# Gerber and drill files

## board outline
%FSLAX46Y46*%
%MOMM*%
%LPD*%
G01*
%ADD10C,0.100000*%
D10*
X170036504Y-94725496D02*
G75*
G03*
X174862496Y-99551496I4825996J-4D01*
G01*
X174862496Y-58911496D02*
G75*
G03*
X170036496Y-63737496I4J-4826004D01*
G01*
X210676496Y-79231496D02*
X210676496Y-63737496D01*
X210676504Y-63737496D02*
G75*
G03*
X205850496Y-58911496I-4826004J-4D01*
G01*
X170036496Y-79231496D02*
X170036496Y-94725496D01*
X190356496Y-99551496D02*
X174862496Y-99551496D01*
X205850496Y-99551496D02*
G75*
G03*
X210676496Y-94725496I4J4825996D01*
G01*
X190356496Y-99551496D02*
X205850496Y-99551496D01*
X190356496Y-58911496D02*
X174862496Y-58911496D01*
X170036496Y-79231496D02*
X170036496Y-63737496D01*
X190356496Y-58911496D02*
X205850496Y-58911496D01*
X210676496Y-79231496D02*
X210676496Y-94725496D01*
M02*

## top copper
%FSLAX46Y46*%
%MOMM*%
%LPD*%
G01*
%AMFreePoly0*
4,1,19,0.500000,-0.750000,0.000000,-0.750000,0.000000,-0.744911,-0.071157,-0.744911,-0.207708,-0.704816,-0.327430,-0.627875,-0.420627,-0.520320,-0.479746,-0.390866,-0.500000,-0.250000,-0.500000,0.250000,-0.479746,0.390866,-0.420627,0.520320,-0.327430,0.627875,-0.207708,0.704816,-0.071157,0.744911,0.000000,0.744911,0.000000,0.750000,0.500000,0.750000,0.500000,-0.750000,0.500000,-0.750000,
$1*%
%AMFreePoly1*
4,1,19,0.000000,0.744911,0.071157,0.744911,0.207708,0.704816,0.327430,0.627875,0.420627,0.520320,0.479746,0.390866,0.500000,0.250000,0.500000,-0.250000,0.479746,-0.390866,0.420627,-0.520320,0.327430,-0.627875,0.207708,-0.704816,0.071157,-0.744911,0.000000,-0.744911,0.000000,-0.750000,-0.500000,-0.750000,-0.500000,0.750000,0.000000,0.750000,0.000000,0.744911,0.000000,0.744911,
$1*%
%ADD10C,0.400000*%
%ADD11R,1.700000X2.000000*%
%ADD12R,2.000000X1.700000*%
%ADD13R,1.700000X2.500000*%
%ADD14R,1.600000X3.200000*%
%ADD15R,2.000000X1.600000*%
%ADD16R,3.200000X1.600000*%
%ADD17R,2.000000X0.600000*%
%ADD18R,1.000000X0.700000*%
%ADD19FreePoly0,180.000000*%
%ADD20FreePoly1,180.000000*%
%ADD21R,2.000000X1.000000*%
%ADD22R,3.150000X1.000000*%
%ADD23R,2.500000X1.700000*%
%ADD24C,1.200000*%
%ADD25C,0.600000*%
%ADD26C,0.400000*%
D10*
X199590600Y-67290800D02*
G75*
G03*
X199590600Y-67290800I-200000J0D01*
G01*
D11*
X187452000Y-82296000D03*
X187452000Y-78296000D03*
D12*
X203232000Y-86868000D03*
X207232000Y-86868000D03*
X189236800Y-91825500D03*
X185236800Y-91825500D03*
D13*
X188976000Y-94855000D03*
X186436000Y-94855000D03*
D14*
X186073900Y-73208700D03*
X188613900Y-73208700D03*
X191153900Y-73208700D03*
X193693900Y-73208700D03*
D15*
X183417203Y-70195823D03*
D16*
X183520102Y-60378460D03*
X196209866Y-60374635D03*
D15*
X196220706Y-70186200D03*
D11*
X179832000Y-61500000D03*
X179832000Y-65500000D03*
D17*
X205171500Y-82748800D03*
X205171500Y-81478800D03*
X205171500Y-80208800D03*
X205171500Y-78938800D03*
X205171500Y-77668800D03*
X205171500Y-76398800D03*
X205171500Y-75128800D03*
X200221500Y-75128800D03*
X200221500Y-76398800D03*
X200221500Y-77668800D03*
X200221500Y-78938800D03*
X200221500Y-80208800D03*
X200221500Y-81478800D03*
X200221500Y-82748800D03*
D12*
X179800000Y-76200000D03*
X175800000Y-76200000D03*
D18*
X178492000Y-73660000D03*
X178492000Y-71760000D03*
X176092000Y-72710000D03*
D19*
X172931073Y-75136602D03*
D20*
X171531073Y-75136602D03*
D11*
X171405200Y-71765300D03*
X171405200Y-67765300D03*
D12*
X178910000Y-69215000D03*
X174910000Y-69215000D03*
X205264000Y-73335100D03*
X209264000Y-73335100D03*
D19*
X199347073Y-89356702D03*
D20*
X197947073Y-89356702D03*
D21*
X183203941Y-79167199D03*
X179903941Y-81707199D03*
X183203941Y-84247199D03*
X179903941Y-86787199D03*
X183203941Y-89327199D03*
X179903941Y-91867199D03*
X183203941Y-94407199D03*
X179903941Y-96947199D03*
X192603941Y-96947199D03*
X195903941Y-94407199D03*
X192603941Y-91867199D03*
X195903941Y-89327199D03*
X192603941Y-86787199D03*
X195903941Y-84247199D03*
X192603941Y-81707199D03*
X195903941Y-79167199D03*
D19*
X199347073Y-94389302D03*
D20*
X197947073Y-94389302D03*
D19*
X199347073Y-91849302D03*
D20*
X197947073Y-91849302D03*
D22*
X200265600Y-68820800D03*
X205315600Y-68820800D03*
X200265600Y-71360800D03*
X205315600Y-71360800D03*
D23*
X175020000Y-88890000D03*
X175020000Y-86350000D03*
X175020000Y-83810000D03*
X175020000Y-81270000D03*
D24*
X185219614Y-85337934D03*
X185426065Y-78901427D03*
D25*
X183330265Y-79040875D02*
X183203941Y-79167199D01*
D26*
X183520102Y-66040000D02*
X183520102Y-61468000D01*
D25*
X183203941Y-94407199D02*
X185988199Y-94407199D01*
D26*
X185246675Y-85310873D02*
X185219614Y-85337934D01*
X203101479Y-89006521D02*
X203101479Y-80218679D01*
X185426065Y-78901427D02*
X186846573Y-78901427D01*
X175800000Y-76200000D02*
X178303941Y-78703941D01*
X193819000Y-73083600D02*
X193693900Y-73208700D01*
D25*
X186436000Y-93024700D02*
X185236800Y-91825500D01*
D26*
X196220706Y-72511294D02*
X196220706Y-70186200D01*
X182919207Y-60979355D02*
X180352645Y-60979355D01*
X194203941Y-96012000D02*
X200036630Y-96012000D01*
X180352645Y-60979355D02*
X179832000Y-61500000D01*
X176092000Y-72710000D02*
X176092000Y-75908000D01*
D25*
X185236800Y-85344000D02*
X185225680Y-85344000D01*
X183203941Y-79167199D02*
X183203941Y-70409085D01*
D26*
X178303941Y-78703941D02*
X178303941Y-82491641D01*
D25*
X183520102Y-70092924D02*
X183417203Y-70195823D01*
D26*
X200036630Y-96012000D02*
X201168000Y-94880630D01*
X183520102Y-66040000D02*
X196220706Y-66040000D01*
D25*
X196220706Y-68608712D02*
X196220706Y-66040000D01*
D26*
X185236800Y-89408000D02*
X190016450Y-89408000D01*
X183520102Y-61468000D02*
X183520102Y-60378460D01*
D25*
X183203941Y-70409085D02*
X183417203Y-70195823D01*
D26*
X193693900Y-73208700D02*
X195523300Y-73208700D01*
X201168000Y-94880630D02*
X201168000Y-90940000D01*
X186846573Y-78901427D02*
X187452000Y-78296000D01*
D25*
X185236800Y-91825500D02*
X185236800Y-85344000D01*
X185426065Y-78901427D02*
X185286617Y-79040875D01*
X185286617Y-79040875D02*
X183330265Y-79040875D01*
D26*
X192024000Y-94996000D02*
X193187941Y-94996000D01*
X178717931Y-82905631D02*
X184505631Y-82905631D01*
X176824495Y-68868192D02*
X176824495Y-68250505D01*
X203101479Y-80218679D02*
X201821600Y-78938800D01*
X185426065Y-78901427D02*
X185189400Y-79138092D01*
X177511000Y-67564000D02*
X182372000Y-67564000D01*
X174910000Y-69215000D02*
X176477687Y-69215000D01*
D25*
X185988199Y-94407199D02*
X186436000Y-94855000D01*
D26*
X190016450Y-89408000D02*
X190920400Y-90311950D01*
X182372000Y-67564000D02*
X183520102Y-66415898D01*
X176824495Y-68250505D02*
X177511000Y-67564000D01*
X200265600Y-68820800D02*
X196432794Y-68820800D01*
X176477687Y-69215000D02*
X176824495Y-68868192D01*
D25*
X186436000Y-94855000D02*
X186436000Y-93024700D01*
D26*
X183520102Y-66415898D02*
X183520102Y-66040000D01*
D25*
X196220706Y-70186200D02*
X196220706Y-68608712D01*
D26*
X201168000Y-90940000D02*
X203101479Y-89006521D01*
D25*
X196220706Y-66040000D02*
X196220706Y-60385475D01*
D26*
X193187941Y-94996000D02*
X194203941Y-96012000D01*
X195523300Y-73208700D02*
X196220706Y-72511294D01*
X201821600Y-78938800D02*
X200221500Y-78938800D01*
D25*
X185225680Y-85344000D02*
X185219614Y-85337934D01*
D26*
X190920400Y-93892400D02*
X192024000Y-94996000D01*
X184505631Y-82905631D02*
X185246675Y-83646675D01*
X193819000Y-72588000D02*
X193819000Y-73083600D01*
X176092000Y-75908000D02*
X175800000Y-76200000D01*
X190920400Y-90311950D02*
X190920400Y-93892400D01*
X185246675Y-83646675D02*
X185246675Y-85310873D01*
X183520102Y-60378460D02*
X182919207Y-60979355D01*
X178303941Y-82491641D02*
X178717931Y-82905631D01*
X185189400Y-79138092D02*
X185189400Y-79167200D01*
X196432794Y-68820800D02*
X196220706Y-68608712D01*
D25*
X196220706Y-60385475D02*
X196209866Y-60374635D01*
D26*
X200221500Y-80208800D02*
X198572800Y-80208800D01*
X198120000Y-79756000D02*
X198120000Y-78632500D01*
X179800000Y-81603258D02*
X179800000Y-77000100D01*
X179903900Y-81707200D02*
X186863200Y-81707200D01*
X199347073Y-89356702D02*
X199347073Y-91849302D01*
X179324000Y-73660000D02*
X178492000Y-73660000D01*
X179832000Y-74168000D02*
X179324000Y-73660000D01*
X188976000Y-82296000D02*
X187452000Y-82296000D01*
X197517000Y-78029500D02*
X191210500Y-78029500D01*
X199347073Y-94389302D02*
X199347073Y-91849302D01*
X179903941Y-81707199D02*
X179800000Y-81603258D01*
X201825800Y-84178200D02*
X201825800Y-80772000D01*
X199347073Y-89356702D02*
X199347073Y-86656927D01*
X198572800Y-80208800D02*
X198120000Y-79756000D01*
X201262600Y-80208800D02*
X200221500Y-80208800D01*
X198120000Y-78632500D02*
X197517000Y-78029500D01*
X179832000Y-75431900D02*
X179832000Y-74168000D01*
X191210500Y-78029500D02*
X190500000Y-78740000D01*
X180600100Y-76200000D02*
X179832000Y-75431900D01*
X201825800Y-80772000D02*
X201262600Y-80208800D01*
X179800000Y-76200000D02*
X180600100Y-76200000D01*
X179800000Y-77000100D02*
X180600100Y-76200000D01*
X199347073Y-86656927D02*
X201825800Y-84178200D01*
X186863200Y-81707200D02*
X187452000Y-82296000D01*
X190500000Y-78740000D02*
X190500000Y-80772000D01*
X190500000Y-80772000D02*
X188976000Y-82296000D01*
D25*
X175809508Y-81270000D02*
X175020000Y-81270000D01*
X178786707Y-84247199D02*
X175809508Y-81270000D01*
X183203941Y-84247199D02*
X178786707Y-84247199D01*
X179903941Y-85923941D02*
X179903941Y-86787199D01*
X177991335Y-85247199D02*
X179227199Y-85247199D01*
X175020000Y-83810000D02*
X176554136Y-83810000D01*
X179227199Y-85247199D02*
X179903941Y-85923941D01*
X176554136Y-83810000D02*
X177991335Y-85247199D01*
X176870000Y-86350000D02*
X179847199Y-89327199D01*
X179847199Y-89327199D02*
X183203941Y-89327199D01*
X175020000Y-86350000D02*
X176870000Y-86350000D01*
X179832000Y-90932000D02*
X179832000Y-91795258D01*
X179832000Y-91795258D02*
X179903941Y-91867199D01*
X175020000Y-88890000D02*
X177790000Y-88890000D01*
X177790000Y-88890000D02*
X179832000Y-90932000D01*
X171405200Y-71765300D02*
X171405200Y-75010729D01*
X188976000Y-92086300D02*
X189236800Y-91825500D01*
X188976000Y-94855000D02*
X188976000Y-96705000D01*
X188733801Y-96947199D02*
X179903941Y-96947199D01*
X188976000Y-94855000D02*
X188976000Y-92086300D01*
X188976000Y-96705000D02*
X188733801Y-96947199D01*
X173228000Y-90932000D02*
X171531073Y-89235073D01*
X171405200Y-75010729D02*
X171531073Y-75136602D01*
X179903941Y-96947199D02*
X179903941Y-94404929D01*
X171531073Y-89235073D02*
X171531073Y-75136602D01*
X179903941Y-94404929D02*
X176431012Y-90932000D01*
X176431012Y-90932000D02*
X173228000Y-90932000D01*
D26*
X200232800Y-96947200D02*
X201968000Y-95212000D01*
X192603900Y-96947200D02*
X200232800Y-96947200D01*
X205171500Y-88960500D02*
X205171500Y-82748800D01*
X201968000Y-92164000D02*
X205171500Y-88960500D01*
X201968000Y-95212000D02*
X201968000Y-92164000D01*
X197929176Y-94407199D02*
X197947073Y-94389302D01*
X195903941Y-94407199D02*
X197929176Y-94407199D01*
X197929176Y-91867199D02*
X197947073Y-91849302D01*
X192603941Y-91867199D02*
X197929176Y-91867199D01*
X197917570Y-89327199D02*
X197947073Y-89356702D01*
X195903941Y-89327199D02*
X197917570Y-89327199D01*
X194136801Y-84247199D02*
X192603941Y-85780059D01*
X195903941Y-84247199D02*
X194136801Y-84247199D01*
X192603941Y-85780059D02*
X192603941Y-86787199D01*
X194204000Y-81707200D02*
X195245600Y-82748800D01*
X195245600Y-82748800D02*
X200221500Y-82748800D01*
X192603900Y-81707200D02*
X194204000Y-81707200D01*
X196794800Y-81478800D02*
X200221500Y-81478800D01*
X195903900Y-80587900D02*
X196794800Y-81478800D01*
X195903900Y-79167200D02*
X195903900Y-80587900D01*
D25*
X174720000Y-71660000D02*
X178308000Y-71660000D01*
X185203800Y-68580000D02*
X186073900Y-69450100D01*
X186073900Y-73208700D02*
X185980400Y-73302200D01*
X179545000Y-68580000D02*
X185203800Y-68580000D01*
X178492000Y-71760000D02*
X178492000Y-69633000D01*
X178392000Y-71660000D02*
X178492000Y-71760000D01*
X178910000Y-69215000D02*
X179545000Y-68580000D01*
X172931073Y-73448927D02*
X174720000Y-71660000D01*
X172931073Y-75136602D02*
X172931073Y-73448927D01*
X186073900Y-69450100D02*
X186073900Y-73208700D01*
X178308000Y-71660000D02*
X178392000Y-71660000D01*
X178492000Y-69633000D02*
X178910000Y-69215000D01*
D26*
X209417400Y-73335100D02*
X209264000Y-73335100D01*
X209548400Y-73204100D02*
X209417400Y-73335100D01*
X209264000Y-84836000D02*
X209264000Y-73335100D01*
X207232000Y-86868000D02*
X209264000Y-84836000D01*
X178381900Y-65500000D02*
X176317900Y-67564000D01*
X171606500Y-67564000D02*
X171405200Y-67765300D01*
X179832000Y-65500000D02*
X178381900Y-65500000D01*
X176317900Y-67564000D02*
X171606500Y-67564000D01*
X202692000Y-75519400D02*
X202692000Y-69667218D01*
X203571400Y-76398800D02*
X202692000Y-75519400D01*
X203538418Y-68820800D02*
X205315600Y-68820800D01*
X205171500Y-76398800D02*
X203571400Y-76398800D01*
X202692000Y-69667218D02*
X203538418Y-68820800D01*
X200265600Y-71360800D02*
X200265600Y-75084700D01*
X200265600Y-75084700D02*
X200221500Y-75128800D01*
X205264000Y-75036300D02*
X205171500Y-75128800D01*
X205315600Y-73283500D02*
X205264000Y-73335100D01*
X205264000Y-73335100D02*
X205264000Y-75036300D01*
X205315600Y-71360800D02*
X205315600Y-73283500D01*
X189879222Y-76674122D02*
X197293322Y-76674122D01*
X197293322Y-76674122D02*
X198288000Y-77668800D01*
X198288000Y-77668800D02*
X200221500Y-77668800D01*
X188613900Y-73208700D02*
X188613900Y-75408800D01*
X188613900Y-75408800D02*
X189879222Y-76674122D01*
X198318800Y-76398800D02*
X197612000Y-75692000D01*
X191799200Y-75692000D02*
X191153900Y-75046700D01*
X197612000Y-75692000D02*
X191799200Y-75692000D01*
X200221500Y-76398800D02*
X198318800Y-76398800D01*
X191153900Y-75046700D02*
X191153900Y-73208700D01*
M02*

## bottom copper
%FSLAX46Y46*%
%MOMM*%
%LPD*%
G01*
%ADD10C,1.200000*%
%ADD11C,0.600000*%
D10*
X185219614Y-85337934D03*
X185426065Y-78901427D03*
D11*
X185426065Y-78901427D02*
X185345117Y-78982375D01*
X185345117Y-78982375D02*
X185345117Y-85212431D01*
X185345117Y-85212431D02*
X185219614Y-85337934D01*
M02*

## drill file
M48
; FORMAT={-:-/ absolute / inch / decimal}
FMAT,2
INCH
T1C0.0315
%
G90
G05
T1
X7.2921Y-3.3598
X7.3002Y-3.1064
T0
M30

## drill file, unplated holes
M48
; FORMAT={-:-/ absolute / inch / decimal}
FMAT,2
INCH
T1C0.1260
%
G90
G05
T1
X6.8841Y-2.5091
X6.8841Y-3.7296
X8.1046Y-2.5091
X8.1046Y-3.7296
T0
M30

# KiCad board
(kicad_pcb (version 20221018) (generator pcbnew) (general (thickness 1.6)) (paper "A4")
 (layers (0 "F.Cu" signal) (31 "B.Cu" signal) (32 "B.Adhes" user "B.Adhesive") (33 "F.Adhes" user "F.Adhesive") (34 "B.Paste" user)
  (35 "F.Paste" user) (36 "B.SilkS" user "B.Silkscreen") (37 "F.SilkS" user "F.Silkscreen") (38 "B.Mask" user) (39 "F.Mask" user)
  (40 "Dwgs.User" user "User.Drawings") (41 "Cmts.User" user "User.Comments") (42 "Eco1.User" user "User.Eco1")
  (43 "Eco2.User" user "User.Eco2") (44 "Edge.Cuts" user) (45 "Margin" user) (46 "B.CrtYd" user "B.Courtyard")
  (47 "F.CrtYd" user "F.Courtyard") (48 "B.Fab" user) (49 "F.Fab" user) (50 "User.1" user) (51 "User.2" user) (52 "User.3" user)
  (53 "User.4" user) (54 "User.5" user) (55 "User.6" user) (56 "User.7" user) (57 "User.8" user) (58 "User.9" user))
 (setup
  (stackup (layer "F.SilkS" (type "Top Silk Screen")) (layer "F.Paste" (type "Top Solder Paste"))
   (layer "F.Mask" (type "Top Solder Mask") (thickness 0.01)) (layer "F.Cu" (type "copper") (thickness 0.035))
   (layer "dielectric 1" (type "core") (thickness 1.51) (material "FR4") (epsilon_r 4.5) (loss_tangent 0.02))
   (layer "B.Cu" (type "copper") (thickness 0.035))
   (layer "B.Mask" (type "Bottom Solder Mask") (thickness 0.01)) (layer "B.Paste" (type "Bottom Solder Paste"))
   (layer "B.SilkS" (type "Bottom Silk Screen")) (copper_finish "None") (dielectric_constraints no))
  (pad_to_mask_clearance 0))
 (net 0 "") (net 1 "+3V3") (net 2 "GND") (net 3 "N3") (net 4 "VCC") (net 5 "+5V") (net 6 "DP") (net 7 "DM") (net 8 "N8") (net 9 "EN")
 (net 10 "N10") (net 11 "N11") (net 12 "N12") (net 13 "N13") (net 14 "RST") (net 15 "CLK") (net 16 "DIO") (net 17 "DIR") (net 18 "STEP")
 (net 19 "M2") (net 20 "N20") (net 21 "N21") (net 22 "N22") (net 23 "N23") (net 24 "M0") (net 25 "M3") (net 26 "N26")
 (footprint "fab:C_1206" (layer "F.Cu") (at 187.452 80.296 90)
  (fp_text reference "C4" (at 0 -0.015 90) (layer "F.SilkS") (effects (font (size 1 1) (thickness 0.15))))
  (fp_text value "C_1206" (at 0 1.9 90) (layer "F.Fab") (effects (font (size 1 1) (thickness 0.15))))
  (pad "1" smd rect (at -2 0 90) (size 2 1.7) (layers "F.Cu" "F.Paste" "F.Mask") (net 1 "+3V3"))
  (pad "2" smd rect (at 2 0 90) (size 2 1.7) (layers "F.Cu" "F.Paste" "F.Mask") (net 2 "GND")))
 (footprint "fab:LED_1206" (layer "F.Cu") (at 205.232 86.868)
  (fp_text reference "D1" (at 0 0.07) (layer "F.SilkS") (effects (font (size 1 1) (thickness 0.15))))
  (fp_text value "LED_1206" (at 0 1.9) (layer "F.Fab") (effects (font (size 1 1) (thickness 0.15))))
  (pad "1" smd rect (at -2 0) (size 2 1.7) (layers "F.Cu" "F.Paste" "F.Mask") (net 2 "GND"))
  (pad "2" smd rect (at 2 0) (size 2 1.7) (layers "F.Cu" "F.Paste" "F.Mask") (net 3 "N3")))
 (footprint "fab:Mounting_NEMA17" (layer "F.Cu") (at 190.3565 79.2315)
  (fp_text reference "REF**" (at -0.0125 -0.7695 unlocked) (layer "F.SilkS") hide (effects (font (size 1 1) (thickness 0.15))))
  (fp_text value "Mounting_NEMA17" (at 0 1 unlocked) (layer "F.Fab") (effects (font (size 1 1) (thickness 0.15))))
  (pad "" np_thru_hole circle (at -15.5 -15.5) (size 3.2 3.2) (drill 3.2) (layers "*.Cu" "*.Mask") (clearance 1.9))
  (pad "" np_thru_hole circle (at -15.5 15.5) (size 3.2 3.2) (drill 3.2) (layers "*.Cu" "*.Mask") (clearance 1.9))
  (pad "" np_thru_hole circle (at 15.5 -15.5) (size 3.2 3.2) (drill 3.2) (layers "*.Cu" "*.Mask") (clearance 1.9))
  (pad "" np_thru_hole circle (at 15.5 15.5) (size 3.2 3.2) (drill 3.2) (layers "*.Cu" "*.Mask") (clearance 1.9)))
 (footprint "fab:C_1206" (layer "F.Cu") (at 187.2368 91.8255 180)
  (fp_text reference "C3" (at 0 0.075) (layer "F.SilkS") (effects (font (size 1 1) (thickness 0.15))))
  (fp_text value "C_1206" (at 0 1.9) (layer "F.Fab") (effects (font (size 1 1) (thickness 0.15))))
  (pad "1" smd rect (at -2 0 180) (size 2 1.7) (layers "F.Cu" "F.Paste" "F.Mask") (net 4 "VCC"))
  (pad "2" smd rect (at 2 0 180) (size 2 1.7) (layers "F.Cu" "F.Paste" "F.Mask") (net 2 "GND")))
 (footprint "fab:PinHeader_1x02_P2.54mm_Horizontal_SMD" (layer "F.Cu") (at 188.976 94.855 -90)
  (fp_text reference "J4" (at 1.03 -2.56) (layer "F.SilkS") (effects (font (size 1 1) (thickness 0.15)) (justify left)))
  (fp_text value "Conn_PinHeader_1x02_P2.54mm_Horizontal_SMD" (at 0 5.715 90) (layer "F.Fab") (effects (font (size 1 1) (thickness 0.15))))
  (pad "1" smd rect (at 0 0 270) (size 2.5 1.7) (layers "F.Cu" "F.Paste" "F.Mask") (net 4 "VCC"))
  (pad "2" smd rect (at 0 2.54 270) (size 2.5 1.7) (layers "F.Cu" "F.Paste" "F.Mask") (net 2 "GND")))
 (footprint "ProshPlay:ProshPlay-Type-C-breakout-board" (layer "F.Cu") (at 189.8689 73.1962)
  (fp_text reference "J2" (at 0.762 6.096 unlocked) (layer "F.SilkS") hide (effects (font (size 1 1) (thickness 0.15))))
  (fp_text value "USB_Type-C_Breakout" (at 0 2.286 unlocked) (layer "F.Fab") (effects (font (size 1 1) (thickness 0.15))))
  (pad "1" smd rect (at -3.795 0.0125 90) (size 3.2 1.6) (layers "F.Cu" "F.Paste" "F.Mask") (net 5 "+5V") (thermal_bridge_angle 45))
  (pad "2" smd rect (at -1.255 0.0125 90) (size 3.2 1.6) (layers "F.Cu" "F.Paste" "F.Mask") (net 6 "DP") (thermal_bridge_angle 45))
  (pad "3" smd rect (at 1.285 0.0125 90) (size 3.2 1.6) (layers "F.Cu" "F.Paste" "F.Mask") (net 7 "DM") (thermal_bridge_angle 45))
  (pad "4" smd rect (at 3.825 0.0125 90) (size 3.2 1.6) (layers "F.Cu" "F.Paste" "F.Mask") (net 2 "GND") (thermal_bridge_angle 45))
  (pad "5" smd rect (at -6.451697 -3.000377 180) (size 2 1.6) (layers "F.Cu" "F.Paste" "F.Mask") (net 2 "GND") (thermal_bridge_angle 45))
  (pad "5" smd rect (at -6.348798 -12.81774 180) (size 3.2 1.6) (layers "F.Cu" "F.Paste" "F.Mask") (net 2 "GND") (thermal_bridge_angle 45))
  (pad "5" smd rect (at 6.340966 -12.821565 180) (size 3.2 1.6) (layers "F.Cu" "F.Paste" "F.Mask") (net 2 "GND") (thermal_bridge_angle 45))
  (pad "5" smd rect (at 6.351806 -3.01 180) (size 2 1.6) (layers "F.Cu" "F.Paste" "F.Mask") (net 2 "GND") (thermal_bridge_angle 45))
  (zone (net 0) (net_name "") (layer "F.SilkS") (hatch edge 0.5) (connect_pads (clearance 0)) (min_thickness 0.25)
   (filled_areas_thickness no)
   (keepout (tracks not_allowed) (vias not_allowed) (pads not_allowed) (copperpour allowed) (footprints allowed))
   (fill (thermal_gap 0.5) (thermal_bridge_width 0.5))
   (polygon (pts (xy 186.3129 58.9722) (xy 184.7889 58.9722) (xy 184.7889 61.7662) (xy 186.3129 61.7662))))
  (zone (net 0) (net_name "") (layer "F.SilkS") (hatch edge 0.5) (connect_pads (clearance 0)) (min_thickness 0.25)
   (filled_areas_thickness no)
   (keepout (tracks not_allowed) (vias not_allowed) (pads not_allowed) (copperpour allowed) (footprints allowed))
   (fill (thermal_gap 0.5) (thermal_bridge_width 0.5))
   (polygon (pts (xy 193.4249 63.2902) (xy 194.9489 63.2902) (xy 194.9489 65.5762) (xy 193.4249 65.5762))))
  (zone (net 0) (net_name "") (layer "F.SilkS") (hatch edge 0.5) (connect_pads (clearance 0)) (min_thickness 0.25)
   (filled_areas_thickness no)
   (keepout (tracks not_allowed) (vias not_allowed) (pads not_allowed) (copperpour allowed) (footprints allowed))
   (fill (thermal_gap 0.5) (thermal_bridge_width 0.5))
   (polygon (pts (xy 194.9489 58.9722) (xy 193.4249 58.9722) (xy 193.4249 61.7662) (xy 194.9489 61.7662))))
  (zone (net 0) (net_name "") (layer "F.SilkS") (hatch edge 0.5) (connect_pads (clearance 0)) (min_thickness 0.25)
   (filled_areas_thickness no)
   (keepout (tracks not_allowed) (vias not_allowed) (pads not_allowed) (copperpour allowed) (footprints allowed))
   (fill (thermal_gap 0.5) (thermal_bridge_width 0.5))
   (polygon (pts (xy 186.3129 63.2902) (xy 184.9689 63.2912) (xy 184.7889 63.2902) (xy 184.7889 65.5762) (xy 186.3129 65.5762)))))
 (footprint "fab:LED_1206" (layer "F.Cu") (at 179.832 63.5 -90)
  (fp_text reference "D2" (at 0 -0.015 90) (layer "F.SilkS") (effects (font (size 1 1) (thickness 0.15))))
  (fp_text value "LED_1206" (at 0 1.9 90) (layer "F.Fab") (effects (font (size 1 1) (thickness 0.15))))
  (pad "1" smd rect (at -2 0 270) (size 2 1.7) (layers "F.Cu" "F.Paste" "F.Mask") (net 2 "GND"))
  (pad "2" smd rect (at 2 0 270) (size 2 1.7) (layers "F.Cu" "F.Paste" "F.Mask") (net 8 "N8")))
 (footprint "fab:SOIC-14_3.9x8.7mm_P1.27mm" (layer "F.Cu") (at 202.6965 78.9388 180)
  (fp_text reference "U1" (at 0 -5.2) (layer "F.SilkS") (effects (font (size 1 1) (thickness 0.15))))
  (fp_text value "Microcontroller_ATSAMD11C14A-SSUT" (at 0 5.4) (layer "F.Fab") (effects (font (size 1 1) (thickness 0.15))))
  (pad "1" smd rect (at -2.475 -3.81 180) (size 2 0.6) (layers "F.Cu" "F.Paste" "F.Mask") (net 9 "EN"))
  (pad "2" smd rect (at -2.475 -2.54 180) (size 2 0.6) (layers "F.Cu" "F.Paste" "F.Mask") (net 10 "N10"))
  (pad "3" smd rect (at -2.475 -1.27 180) (size 2 0.6) (layers "F.Cu" "F.Paste" "F.Mask") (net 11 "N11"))
  (pad "4" smd rect (at -2.475 0 180) (size 2 0.6) (layers "F.Cu" "F.Paste" "F.Mask") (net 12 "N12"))
  (pad "5" smd rect (at -2.475 1.27 180) (size 2 0.6) (layers "F.Cu" "F.Paste" "F.Mask") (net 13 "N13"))
  (pad "6" smd rect (at -2.475 2.54 180) (size 2 0.6) (layers "F.Cu" "F.Paste" "F.Mask") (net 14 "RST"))
  (pad "7" smd rect (at -2.475 3.81 180) (size 2 0.6) (layers "F.Cu" "F.Paste" "F.Mask") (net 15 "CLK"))
  (pad "8" smd rect (at 2.475 3.81 180) (size 2 0.6) (layers "F.Cu" "F.Paste" "F.Mask") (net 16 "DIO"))
  (pad "9" smd rect (at 2.475 2.54 180) (size 2 0.6) (layers "F.Cu" "F.Paste" "F.Mask") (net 7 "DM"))
  (pad "10" smd rect (at 2.475 1.27 180) (size 2 0.6) (layers "F.Cu" "F.Paste" "F.Mask") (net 6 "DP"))
  (pad "11" smd rect (at 2.475 0 180) (size 2 0.6) (layers "F.Cu" "F.Paste" "F.Mask") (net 2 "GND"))
  (pad "12" smd rect (at 2.475 -1.27 180) (size 2 0.6) (layers "F.Cu" "F.Paste" "F.Mask") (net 1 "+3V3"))
  (pad "13" smd rect (at 2.475 -2.54 180) (size 2 0.6) (layers "F.Cu" "F.Paste" "F.Mask") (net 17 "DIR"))
  (pad "14" smd rect (at 2.475 -3.81 180) (size 2 0.6) (layers "F.Cu" "F.Paste" "F.Mask") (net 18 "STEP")))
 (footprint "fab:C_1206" (layer "F.Cu") (at 177.8 76.2 180)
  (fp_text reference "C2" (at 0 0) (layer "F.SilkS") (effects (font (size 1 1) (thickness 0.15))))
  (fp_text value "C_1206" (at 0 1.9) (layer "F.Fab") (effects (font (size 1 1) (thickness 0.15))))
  (pad "1" smd rect (at -2 0 180) (size 2 1.7) (layers "F.Cu" "F.Paste" "F.Mask") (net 1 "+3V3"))
  (pad "2" smd rect (at 2 0 180) (size 2 1.7) (layers "F.Cu" "F.Paste" "F.Mask") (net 2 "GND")))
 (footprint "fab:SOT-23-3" (layer "F.Cu") (at 177.292 72.71 180)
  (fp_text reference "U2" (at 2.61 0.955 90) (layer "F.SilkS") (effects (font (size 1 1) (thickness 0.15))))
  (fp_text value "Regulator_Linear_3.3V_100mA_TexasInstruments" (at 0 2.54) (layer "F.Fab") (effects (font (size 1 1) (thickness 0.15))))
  (pad "1" smd rect (at -1.2 -0.95 180) (size 1 0.7) (layers "F.Cu" "F.Paste" "F.Mask") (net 1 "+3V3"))
  (pad "2" smd rect (at -1.2 0.95 180) (size 1 0.7) (layers "F.Cu" "F.Paste" "F.Mask") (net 5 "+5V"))
  (pad "3" smd rect (at 1.2 0 180) (size 1 0.7) (layers "F.Cu" "F.Paste" "F.Mask") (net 2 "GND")))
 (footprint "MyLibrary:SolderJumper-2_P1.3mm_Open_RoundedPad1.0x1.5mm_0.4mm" (layer "F.Cu") (at 172.212 75.184 180)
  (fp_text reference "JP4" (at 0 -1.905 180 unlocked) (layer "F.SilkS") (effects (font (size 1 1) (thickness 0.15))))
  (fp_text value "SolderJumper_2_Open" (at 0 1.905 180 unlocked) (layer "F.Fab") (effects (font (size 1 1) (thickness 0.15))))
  (pad "1" smd custom (at -0.719073 0.047398 180) (size 1 0.5) (layers "F.Cu" "F.Mask") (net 5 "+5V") (zone_connect 2)
   (thermal_bridge_angle 45) (options (clearance outline) (anchor rect)) (primitives))
  (pad "2" smd custom (at 0.680927 0.047398 180) (size 1 0.5) (layers "F.Cu" "F.Mask") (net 4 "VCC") (zone_connect 2)
   (thermal_bridge_angle 45) (options (clearance outline) (anchor rect)) (primitives)))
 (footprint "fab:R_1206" (layer "F.Cu") (at 171.4052 69.7653 90)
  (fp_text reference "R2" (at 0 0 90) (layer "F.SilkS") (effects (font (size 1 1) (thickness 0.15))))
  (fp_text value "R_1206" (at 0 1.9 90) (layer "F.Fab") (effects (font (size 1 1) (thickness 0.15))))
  (pad "1" smd rect (at -2 0 90) (size 2 1.7) (layers "F.Cu" "F.Paste" "F.Mask") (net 4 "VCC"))
  (pad "2" smd rect (at 2 0 90) (size 2 1.7) (layers "F.Cu" "F.Paste" "F.Mask") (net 8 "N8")))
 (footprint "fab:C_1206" (layer "F.Cu") (at 176.91 69.215 180)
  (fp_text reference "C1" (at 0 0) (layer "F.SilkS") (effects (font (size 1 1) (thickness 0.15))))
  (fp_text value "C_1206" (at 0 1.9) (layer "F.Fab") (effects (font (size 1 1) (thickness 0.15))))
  (pad "1" smd rect (at -2 0 180) (size 2 1.7) (layers "F.Cu" "F.Paste" "F.Mask") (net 5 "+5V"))
  (pad "2" smd rect (at 2 0 180) (size 2 1.7) (layers "F.Cu" "F.Paste" "F.Mask") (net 2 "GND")))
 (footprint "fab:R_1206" (layer "F.Cu") (at 207.264 73.3351)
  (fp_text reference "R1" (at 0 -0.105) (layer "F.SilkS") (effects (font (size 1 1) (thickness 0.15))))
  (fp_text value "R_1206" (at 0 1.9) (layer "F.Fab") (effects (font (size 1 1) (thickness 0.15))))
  (pad "1" smd rect (at -2 0) (size 2 1.7) (layers "F.Cu" "F.Paste" "F.Mask") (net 15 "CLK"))
  (pad "2" smd rect (at 2 0) (size 2 1.7) (layers "F.Cu" "F.Paste" "F.Mask") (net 3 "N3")))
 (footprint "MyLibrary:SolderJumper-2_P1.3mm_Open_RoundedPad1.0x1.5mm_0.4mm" (layer "F.Cu") (at 198.628 89.4041 180)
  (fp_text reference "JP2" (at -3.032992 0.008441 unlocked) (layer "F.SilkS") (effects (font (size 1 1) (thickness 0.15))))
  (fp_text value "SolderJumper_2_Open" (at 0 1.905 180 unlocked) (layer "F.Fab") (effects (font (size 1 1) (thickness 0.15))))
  (pad "1" smd custom (at -0.719073 0.047398 180) (size 1 0.5) (layers "F.Cu" "F.Mask") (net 1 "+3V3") (zone_connect 2)
   (thermal_bridge_angle 45) (options (clearance outline) (anchor rect)) (primitives))
  (pad "2" smd custom (at 0.680927 0.047398 180) (size 1 0.5) (layers "F.Cu" "F.Mask") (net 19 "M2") (zone_connect 2)
   (thermal_bridge_angle 45) (options (clearance outline) (anchor rect)) (primitives)))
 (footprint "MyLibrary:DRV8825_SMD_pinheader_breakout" (layer "F.Cu") (at 187.7853 88.0572)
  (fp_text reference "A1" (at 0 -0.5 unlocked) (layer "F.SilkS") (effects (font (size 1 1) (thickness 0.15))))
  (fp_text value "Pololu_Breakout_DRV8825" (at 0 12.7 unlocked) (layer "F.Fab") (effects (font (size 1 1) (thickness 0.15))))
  (pad "1" smd rect (at -4.581359 -8.890001) (size 2 1) (layers "F.Cu" "F.Paste" "F.Mask") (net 2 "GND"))
  (pad "2" smd rect (at -7.881359 -6.350001) (size 2 1) (layers "F.Cu" "F.Paste" "F.Mask") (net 1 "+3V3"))
  (pad "3" smd rect (at -4.581359 -3.810001) (size 2 1) (layers "F.Cu" "F.Paste" "F.Mask") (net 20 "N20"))
  (pad "4" smd rect (at -7.881359 -1.270001) (size 2 1) (layers "F.Cu" "F.Paste" "F.Mask") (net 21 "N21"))
  (pad "5" smd rect (at -4.581359 1.269999) (size 2 1) (layers "F.Cu" "F.Paste" "F.Mask") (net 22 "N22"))
  (pad "6" smd rect (at -7.881359 3.809999) (size 2 1) (layers "F.Cu" "F.Paste" "F.Mask") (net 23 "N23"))
  (pad "7" smd rect (at -4.581359 6.349999) (size 2 1) (layers "F.Cu" "F.Paste" "F.Mask") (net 2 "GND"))
  (pad "8" smd rect (at -7.881359 8.889999) (size 2 1) (layers "F.Cu" "F.Paste" "F.Mask") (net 4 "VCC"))
  (pad "9" smd rect (at 4.818641 8.889999) (size 2 1) (layers "F.Cu" "F.Paste" "F.Mask") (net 9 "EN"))
  (pad "10" smd rect (at 8.118641 6.349999) (size 2 1) (layers "F.Cu" "F.Paste" "F.Mask") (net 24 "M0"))
  (pad "11" smd rect (at 4.818641 3.809999) (size 2 1) (layers "F.Cu" "F.Paste" "F.Mask") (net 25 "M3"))
  (pad "12" smd rect (at 8.118641 1.269999) (size 2 1) (layers "F.Cu" "F.Paste" "F.Mask") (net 19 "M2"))
  (pad "13" smd rect (at 4.818641 -1.270001) (size 2 1) (layers "F.Cu" "F.Paste" "F.Mask") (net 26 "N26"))
  (pad "14" smd rect (at 8.118641 -3.810001) (size 2 1) (layers "F.Cu" "F.Paste" "F.Mask") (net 26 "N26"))
  (pad "15" smd rect (at 4.818641 -6.350001) (size 2 1) (layers "F.Cu" "F.Paste" "F.Mask") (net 18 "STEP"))
  (pad "16" smd rect (at 8.118641 -8.890001) (size 2 1) (layers "F.Cu" "F.Paste" "F.Mask") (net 17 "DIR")))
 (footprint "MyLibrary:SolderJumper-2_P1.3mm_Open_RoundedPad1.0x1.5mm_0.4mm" (layer "F.Cu") (at 198.628 94.4367 180)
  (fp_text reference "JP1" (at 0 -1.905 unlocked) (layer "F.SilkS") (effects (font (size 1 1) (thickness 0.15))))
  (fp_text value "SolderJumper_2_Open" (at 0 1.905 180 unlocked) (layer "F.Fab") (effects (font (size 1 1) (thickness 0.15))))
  (pad "1" smd custom (at -0.719073 0.047398 180) (size 1 0.5) (layers "F.Cu" "F.Mask") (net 1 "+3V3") (zone_connect 2)
   (thermal_bridge_angle 45) (options (clearance outline) (anchor rect)) (primitives))
  (pad "2" smd custom (at 0.680927 0.047398 180) (size 1 0.5) (layers "F.Cu" "F.Mask") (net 24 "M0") (zone_connect 2)
   (thermal_bridge_angle 45) (options (clearance outline) (anchor rect)) (primitives)))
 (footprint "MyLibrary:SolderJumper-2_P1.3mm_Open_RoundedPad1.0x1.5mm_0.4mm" (layer "F.Cu") (at 198.628 91.8967 180)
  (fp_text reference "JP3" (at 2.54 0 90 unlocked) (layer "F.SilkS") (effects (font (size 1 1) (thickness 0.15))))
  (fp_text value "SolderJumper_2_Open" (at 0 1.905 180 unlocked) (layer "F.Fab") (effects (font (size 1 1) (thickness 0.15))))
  (pad "1" smd custom (at -0.719073 0.047398 180) (size 1 0.5) (layers "F.Cu" "F.Mask") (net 1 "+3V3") (zone_connect 2)
   (thermal_bridge_angle 45) (options (clearance outline) (anchor rect)) (primitives))
  (pad "2" smd custom (at 0.680927 0.047398 180) (size 1 0.5) (layers "F.Cu" "F.Mask") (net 25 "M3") (zone_connect 2)
   (thermal_bridge_angle 45) (options (clearance outline) (anchor rect)) (primitives)))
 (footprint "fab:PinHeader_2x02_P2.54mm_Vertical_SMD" (layer "F.Cu") (at 202.7906 70.0908)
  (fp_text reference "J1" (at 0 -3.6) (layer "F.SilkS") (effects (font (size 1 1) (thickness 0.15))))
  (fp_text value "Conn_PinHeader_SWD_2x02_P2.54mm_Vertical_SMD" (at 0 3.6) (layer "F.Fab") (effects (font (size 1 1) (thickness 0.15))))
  (fp_circle (center -3.4 -2.8) (end -3.1 -2.8) (stroke (width 0.2) (type solid)) (fill solid) (layer "F.Cu"))
  (pad "1" smd rect (at -2.525 -1.27) (size 3.15 1) (layers "F.Cu" "F.Paste" "F.Mask") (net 2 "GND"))
  (pad "2" smd rect (at 2.525 -1.27) (size 3.15 1) (layers "F.Cu" "F.Paste" "F.Mask") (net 14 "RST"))
  (pad "3" smd rect (at -2.525 1.27) (size 3.15 1) (layers "F.Cu" "F.Paste" "F.Mask") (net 16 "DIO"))
  (pad "4" smd rect (at 2.525 1.27) (size 3.15 1) (layers "F.Cu" "F.Paste" "F.Mask") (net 15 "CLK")))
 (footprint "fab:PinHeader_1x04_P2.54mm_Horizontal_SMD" (layer "F.Cu") (at 175.02 88.89 180)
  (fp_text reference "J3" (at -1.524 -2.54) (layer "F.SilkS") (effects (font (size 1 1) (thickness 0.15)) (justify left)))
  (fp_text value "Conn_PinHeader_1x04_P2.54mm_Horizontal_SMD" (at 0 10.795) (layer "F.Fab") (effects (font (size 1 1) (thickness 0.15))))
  (pad "1" smd rect (at 0 0 180) (size 2.5 1.7) (layers "F.Cu" "F.Paste" "F.Mask") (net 23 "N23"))
  (pad "2" smd rect (at 0 2.54 180) (size 2.5 1.7) (layers "F.Cu" "F.Paste" "F.Mask") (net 22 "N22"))
  (pad "3" smd rect (at 0 5.08 180) (size 2.5 1.7) (layers "F.Cu" "F.Paste" "F.Mask") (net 21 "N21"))
  (pad "4" smd rect (at 0 7.62 180) (size 2.5 1.7) (layers "F.Cu" "F.Paste" "F.Mask") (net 20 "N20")))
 (gr_arc (start 174.862496 99.551496) (mid 171.449999 98.137993) (end 170.036496 94.725496) (stroke (width 0.1) (type default))
  (layer "Edge.Cuts"))
 (gr_arc (start 170.036496 63.737496) (mid 171.449999 60.324999) (end 174.862496 58.911496) (stroke (width 0.1) (type default))
  (layer "Edge.Cuts"))
 (gr_line (start 210.676496 79.231496) (end 210.676496 63.737496) (stroke (width 0.1) (type default)) (layer "Edge.Cuts"))
 (gr_arc (start 205.850496 58.911496) (mid 209.262997 60.324997) (end 210.676496 63.737496) (stroke (width 0.1) (type default))
  (layer "Edge.Cuts"))
 (gr_line (start 170.036496 79.231496) (end 170.036496 94.725496) (stroke (width 0.1) (type default)) (layer "Edge.Cuts"))
 (gr_line (start 190.356496 99.551496) (end 174.862496 99.551496) (stroke (width 0.1) (type default)) (layer "Edge.Cuts"))
 (gr_arc (start 210.676496 94.725496) (mid 209.262994 98.137994) (end 205.850496 99.551496) (stroke (width 0.1) (type default))
  (layer "Edge.Cuts"))
 (gr_line (start 190.356496 99.551496) (end 205.850496 99.551496) (stroke (width 0.1) (type default)) (layer "Edge.Cuts"))
 (gr_line (start 190.356496 58.911496) (end 174.862496 58.911496) (stroke (width 0.1) (type default)) (layer "Edge.Cuts"))
 (gr_line (start 170.036496 79.231496) (end 170.036496 63.737496) (stroke (width 0.1) (type default)) (layer "Edge.Cuts"))
 (gr_line (start 190.356496 58.911496) (end 205.850496 58.911496) (stroke (width 0.1) (type default)) (layer "Edge.Cuts"))
 (gr_line (start 210.676496 79.231496) (end 210.676496 94.725496) (stroke (width 0.1) (type default)) (layer "Edge.Cuts"))
 (segment (start 183.330265 79.040875) (end 183.203941 79.167199) (width 0.6) (layer "F.Cu") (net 2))
 (segment (start 183.520102 66.04) (end 183.520102 61.468) (width 0.4) (layer "F.Cu") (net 2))
 (segment (start 183.203941 94.407199) (end 185.988199 94.407199) (width 0.6) (layer "F.Cu") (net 2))
 (segment (start 185.246675 85.310873) (end 185.219614 85.337934) (width 0.4) (layer "F.Cu") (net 2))
 (segment (start 203.101479 89.006521) (end 203.101479 80.218679) (width 0.4) (layer "F.Cu") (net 2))
 (segment (start 185.426065 78.901427) (end 186.846573 78.901427) (width 0.4) (layer "F.Cu") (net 2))
 (segment (start 175.8 76.2) (end 178.303941 78.703941) (width 0.4) (layer "F.Cu") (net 2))
 (segment (start 193.819 73.0836) (end 193.6939 73.2087) (width 0.4) (layer "F.Cu") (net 2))
 (segment (start 186.436 93.0247) (end 185.2368 91.8255) (width 0.6) (layer "F.Cu") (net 2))
 (segment (start 196.220706 72.511294) (end 196.220706 70.1862) (width 0.4) (layer "F.Cu") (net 2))
 (segment (start 182.919207 60.979355) (end 180.352645 60.979355) (width 0.4) (layer "F.Cu") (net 2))
 (segment (start 194.203941 96.012) (end 200.03663 96.012) (width 0.4) (layer "F.Cu") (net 2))
 (segment (start 180.352645 60.979355) (end 179.832 61.5) (width 0.4) (layer "F.Cu") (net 2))
 (segment (start 176.092 72.71) (end 176.092 75.908) (width 0.4) (layer "F.Cu") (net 2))
 (segment (start 185.2368 85.344) (end 185.22568 85.344) (width 0.6) (layer "F.Cu") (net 2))
 (segment (start 183.203941 79.167199) (end 183.203941 70.409085) (width 0.6) (layer "F.Cu") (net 2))
 (segment (start 178.303941 78.703941) (end 178.303941 82.491641) (width 0.4) (layer "F.Cu") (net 2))
 (segment (start 183.520102 70.092924) (end 183.417203 70.195823) (width 0.6) (layer "F.Cu") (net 2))
 (segment (start 200.03663 96.012) (end 201.168 94.88063) (width 0.4) (layer "F.Cu") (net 2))
 (segment (start 183.520102 66.04) (end 196.220706 66.04) (width 0.4) (layer "F.Cu") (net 2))
 (segment (start 196.220706 68.608712) (end 196.220706 66.04) (width 0.6) (layer "F.Cu") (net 2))
 (segment (start 185.2368 89.408) (end 190.01645 89.408) (width 0.4) (layer "F.Cu") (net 2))
 (segment (start 183.520102 61.468) (end 183.520102 60.37846) (width 0.4) (layer "F.Cu") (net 2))
 (segment (start 183.203941 70.409085) (end 183.417203 70.195823) (width 0.6) (layer "F.Cu") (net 2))
 (segment (start 193.6939 73.2087) (end 195.5233 73.2087) (width 0.4) (layer "F.Cu") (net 2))
 (segment (start 201.168 94.88063) (end 201.168 90.94) (width 0.4) (layer "F.Cu") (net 2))
 (segment (start 186.846573 78.901427) (end 187.452 78.296) (width 0.4) (layer "F.Cu") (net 2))
 (segment (start 185.2368 91.8255) (end 185.2368 85.344) (width 0.6) (layer "F.Cu") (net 2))
 (segment (start 185.426065 78.901427) (end 185.286617 79.040875) (width 0.6) (layer "F.Cu") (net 2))
 (segment (start 185.286617 79.040875) (end 183.330265 79.040875) (width 0.6) (layer "F.Cu") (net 2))
 (segment (start 192.024 94.996) (end 193.187941 94.996) (width 0.4) (layer "F.Cu") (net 2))
 (segment (start 178.717931 82.905631) (end 184.505631 82.905631) (width 0.4) (layer "F.Cu") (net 2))
 (segment (start 176.824495 68.868192) (end 176.824495 68.250505) (width 0.4) (layer "F.Cu") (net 2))
 (segment (start 203.101479 80.218679) (end 201.8216 78.9388) (width 0.4) (layer "F.Cu") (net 2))
 (segment (start 185.426065 78.901427) (end 185.1894 79.138092) (width 0.4) (layer "F.Cu") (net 2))
 (segment (start 177.511 67.564) (end 182.372 67.564) (width 0.4) (layer "F.Cu") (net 2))
 (segment (start 174.91 69.215) (end 176.477687 69.215) (width 0.4) (layer "F.Cu") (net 2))
 (segment (start 185.988199 94.407199) (end 186.436 94.855) (width 0.6) (layer "F.Cu") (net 2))
 (segment (start 190.01645 89.408) (end 190.9204 90.31195) (width 0.4) (layer "F.Cu") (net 2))
 (segment (start 182.372 67.564) (end 183.520102 66.415898) (width 0.4) (layer "F.Cu") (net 2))
 (segment (start 176.824495 68.250505) (end 177.511 67.564) (width 0.4) (layer "F.Cu") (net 2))
 (segment (start 200.2656 68.8208) (end 196.432794 68.8208) (width 0.4) (layer "F.Cu") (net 2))
 (segment (start 176.477687 69.215) (end 176.824495 68.868192) (width 0.4) (layer "F.Cu") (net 2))
 (segment (start 186.436 94.855) (end 186.436 93.0247) (width 0.6) (layer "F.Cu") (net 2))
 (segment (start 183.520102 66.415898) (end 183.520102 66.04) (width 0.4) (layer "F.Cu") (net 2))
 (segment (start 196.220706 70.1862) (end 196.220706 68.608712) (width 0.6) (layer "F.Cu") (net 2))
 (segment (start 201.168 90.94) (end 203.101479 89.006521) (width 0.4) (layer "F.Cu") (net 2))
 (segment (start 196.220706 66.04) (end 196.220706 60.385475) (width 0.6) (layer "F.Cu") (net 2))
 (segment (start 193.187941 94.996) (end 194.203941 96.012) (width 0.4) (layer "F.Cu") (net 2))
 (segment (start 195.5233 73.2087) (end 196.220706 72.511294) (width 0.4) (layer "F.Cu") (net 2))
 (segment (start 201.8216 78.9388) (end 200.2215 78.9388) (width 0.4) (layer "F.Cu") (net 2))
 (segment (start 185.22568 85.344) (end 185.219614 85.337934) (width 0.6) (layer "F.Cu") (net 2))
 (segment (start 190.9204 93.8924) (end 192.024 94.996) (width 0.4) (layer "F.Cu") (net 2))
 (segment (start 184.505631 82.905631) (end 185.246675 83.646675) (width 0.4) (layer "F.Cu") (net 2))
 (segment (start 193.819 72.588) (end 193.819 73.0836) (width 0.4) (layer "F.Cu") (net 2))
 (segment (start 176.092 75.908) (end 175.8 76.2) (width 0.4) (layer "F.Cu") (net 2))
 (segment (start 190.9204 90.31195) (end 190.9204 93.8924) (width 0.4) (layer "F.Cu") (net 2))
 (segment (start 185.246675 83.646675) (end 185.246675 85.310873) (width 0.4) (layer "F.Cu") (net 2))
 (segment (start 183.520102 60.37846) (end 182.919207 60.979355) (width 0.4) (layer "F.Cu") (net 2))
 (segment (start 178.303941 82.491641) (end 178.717931 82.905631) (width 0.4) (layer "F.Cu") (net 2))
 (segment (start 185.1894 79.138092) (end 185.1894 79.1672) (width 0.4) (layer "F.Cu") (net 2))
 (segment (start 196.432794 68.8208) (end 196.220706 68.608712) (width 0.4) (layer "F.Cu") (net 2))
 (segment (start 196.220706 60.385475) (end 196.209866 60.374635) (width 0.6) (layer "F.Cu") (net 2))
 (via (at 185.219614 85.337934) (size 1.2) (drill 0.8) (layers "F.Cu" "B.Cu") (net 2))
 (via (at 185.426065 78.901427) (size 1.2) (drill 0.8) (layers "F.Cu" "B.Cu") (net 2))
 (segment (start 185.426065 78.901427) (end 185.345117 78.982375) (width 0.6) (layer "B.Cu") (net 2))
 (segment (start 185.345117 78.982375) (end 185.345117 85.212431) (width 0.6) (layer "B.Cu") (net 2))
 (segment (start 185.345117 85.212431) (end 185.219614 85.337934) (width 0.6) (layer "B.Cu") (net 2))
 (segment (start 200.2215 80.2088) (end 198.5728 80.2088) (width 0.4) (layer "F.Cu") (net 1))
 (segment (start 198.12 79.756) (end 198.12 78.6325) (width 0.4) (layer "F.Cu") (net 1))
 (segment (start 179.8 81.603258) (end 179.8 77.0001) (width 0.4) (layer "F.Cu") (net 1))
 (segment (start 179.9039 81.7072) (end 186.8632 81.7072) (width 0.4) (layer "F.Cu") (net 1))
 (segment (start 199.347073 89.356702) (end 199.347073 91.849302) (width 0.4) (layer "F.Cu") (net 1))
 (segment (start 179.324 73.66) (end 178.492 73.66) (width 0.4) (layer "F.Cu") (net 1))
 (segment (start 179.832 74.168) (end 179.324 73.66) (width 0.4) (layer "F.Cu") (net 1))
 (segment (start 188.976 82.296) (end 187.452 82.296) (width 0.4) (layer "F.Cu") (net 1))
 (segment (start 197.517 78.0295) (end 191.2105 78.0295) (width 0.4) (layer "F.Cu") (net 1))
 (segment (start 199.347073 94.389302) (end 199.347073 91.849302) (width 0.4) (layer "F.Cu") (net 1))
 (segment (start 179.903941 81.707199) (end 179.8 81.603258) (width 0.4) (layer "F.Cu") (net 1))
 (segment (start 201.8258 84.1782) (end 201.8258 80.772) (width 0.4) (layer "F.Cu") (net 1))
 (segment (start 199.347073 89.356702) (end 199.347073 86.656927) (width 0.4) (layer "F.Cu") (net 1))
 (segment (start 198.5728 80.2088) (end 198.12 79.756) (width 0.4) (layer "F.Cu") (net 1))
 (segment (start 201.2626 80.2088) (end 200.2215 80.2088) (width 0.4) (layer "F.Cu") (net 1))
 (segment (start 198.12 78.6325) (end 197.517 78.0295) (width 0.4) (layer "F.Cu") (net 1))
 (segment (start 179.832 75.4319) (end 179.832 74.168) (width 0.4) (layer "F.Cu") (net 1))
 (segment (start 191.2105 78.0295) (end 190.5 78.74) (width 0.4) (layer "F.Cu") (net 1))
 (segment (start 180.6001 76.2) (end 179.832 75.4319) (width 0.4) (layer "F.Cu") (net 1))
 (segment (start 201.8258 80.772) (end 201.2626 80.2088) (width 0.4) (layer "F.Cu") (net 1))
 (segment (start 179.8 76.2) (end 180.6001 76.2) (width 0.4) (layer "F.Cu") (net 1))
 (segment (start 179.8 77.0001) (end 180.6001 76.2) (width 0.4) (layer "F.Cu") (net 1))
 (segment (start 199.347073 86.656927) (end 201.8258 84.1782) (width 0.4) (layer "F.Cu") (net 1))
 (segment (start 186.8632 81.7072) (end 187.452 82.296) (width 0.4) (layer "F.Cu") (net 1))
 (segment (start 190.5 78.74) (end 190.5 80.772) (width 0.4) (layer "F.Cu") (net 1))
 (segment (start 190.5 80.772) (end 188.976 82.296) (width 0.4) (layer "F.Cu") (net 1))
 (segment (start 175.809508 81.27) (end 175.02 81.27) (width 0.6) (layer "F.Cu") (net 20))
 (segment (start 178.786707 84.247199) (end 175.809508 81.27) (width 0.6) (layer "F.Cu") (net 20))
 (segment (start 183.203941 84.247199) (end 178.786707 84.247199) (width 0.6) (layer "F.Cu") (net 20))
 (segment (start 179.903941 85.923941) (end 179.903941 86.787199) (width 0.6) (layer "F.Cu") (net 21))
 (segment (start 177.991335 85.247199) (end 179.227199 85.247199) (width 0.6) (layer "F.Cu") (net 21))
 (segment (start 175.02 83.81) (end 176.554136 83.81) (width 0.6) (layer "F.Cu") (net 21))
 (segment (start 179.227199 85.247199) (end 179.903941 85.923941) (width 0.6) (layer "F.Cu") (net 21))
 (segment (start 176.554136 83.81) (end 177.991335 85.247199) (width 0.6) (layer "F.Cu") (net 21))
 (segment (start 176.87 86.35) (end 179.847199 89.327199) (width 0.6) (layer "F.Cu") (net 22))
 (segment (start 179.847199 89.327199) (end 183.203941 89.327199) (width 0.6) (layer "F.Cu") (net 22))
 (segment (start 175.02 86.35) (end 176.87 86.35) (width 0.6) (layer "F.Cu") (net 22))
 (segment (start 179.832 90.932) (end 179.832 91.795258) (width 0.6) (layer "F.Cu") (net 23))
 (segment (start 179.832 91.795258) (end 179.903941 91.867199) (width 0.6) (layer "F.Cu") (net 23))
 (segment (start 175.02 88.89) (end 177.79 88.89) (width 0.6) (layer "F.Cu") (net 23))
 (segment (start 177.79 88.89) (end 179.832 90.932) (width 0.6) (layer "F.Cu") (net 23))
 (segment (start 171.4052 71.7653) (end 171.4052 75.010729) (width 0.6) (layer "F.Cu") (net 4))
 (segment (start 188.976 92.0863) (end 189.2368 91.8255) (width 0.6) (layer "F.Cu") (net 4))
 (segment (start 188.976 94.855) (end 188.976 96.705) (width 0.6) (layer "F.Cu") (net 4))
 (segment (start 188.733801 96.947199) (end 179.903941 96.947199) (width 0.6) (layer "F.Cu") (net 4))
 (segment (start 188.976 94.855) (end 188.976 92.0863) (width 0.6) (layer "F.Cu") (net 4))
 (segment (start 188.976 96.705) (end 188.733801 96.947199) (width 0.6) (layer "F.Cu") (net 4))
 (segment (start 173.228 90.932) (end 171.531073 89.235073) (width 0.6) (layer "F.Cu") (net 4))
 (segment (start 171.4052 75.010729) (end 171.531073 75.136602) (width 0.6) (layer "F.Cu") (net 4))
 (segment (start 179.903941 96.947199) (end 179.903941 94.404929) (width 0.6) (layer "F.Cu") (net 4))
 (segment (start 171.531073 89.235073) (end 171.531073 75.136602) (width 0.6) (layer "F.Cu") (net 4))
 (segment (start 179.903941 94.404929) (end 176.431012 90.932) (width 0.6) (layer "F.Cu") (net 4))
 (segment (start 176.431012 90.932) (end 173.228 90.932) (width 0.6) (layer "F.Cu") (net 4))
 (segment (start 200.2328 96.9472) (end 201.968 95.212) (width 0.4) (layer "F.Cu") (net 9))
 (segment (start 192.6039 96.9472) (end 200.2328 96.9472) (width 0.4) (layer "F.Cu") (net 9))
 (segment (start 205.1715 88.9605) (end 205.1715 82.7488) (width 0.4) (layer "F.Cu") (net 9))
 (segment (start 201.968 92.164) (end 205.1715 88.9605) (width 0.4) (layer "F.Cu") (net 9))
 (segment (start 201.968 95.212) (end 201.968 92.164) (width 0.4) (layer "F.Cu") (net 9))
 (segment (start 197.929176 94.407199) (end 197.947073 94.389302) (width 0.4) (layer "F.Cu") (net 24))
 (segment (start 195.903941 94.407199) (end 197.929176 94.407199) (width 0.4) (layer "F.Cu") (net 24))
 (segment (start 197.929176 91.867199) (end 197.947073 91.849302) (width 0.4) (layer "F.Cu") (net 25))
 (segment (start 192.603941 91.867199) (end 197.929176 91.867199) (width 0.4) (layer "F.Cu") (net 25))
 (segment (start 197.91757 89.327199) (end 197.947073 89.356702) (width 0.4) (layer "F.Cu") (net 19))
 (segment (start 195.903941 89.327199) (end 197.91757 89.327199) (width 0.4) (layer "F.Cu") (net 19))
 (segment (start 194.136801 84.247199) (end 192.603941 85.780059) (width 0.4) (layer "F.Cu") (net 26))
 (segment (start 195.903941 84.247199) (end 194.136801 84.247199) (width 0.4) (layer "F.Cu") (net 26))
 (segment (start 192.603941 85.780059) (end 192.603941 86.787199) (width 0.4) (layer "F.Cu") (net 26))
 (segment (start 194.204 81.7072) (end 195.2456 82.7488) (width 0.4) (layer "F.Cu") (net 18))
 (segment (start 195.2456 82.7488) (end 200.2215 82.7488) (width 0.4) (layer "F.Cu") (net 18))
 (segment (start 192.6039 81.7072) (end 194.204 81.7072) (width 0.4) (layer "F.Cu") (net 18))
 (segment (start 196.7948 81.4788) (end 200.2215 81.4788) (width 0.4) (layer "F.Cu") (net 17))
 (segment (start 195.9039 80.5879) (end 196.7948 81.4788) (width 0.4) (layer "F.Cu") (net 17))
 (segment (start 195.9039 79.1672) (end 195.9039 80.5879) (width 0.4) (layer "F.Cu") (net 17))
 (segment (start 174.72 71.66) (end 178.308 71.66) (width 0.6) (layer "F.Cu") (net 5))
 (segment (start 185.2038 68.58) (end 186.0739 69.4501) (width 0.6) (layer "F.Cu") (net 5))
 (segment (start 186.0739 73.2087) (end 185.9804 73.3022) (width 0.6) (layer "F.Cu") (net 5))
 (segment (start 179.545 68.58) (end 185.2038 68.58) (width 0.6) (layer "F.Cu") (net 5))
 (segment (start 178.492 71.76) (end 178.492 69.633) (width 0.6) (layer "F.Cu") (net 5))
 (segment (start 178.392 71.66) (end 178.492 71.76) (width 0.6) (layer "F.Cu") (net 5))
 (segment (start 178.91 69.215) (end 179.545 68.58) (width 0.6) (layer "F.Cu") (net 5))
 (segment (start 172.931073 73.448927) (end 174.72 71.66) (width 0.6) (layer "F.Cu") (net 5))
 (segment (start 172.931073 75.136602) (end 172.931073 73.448927) (width 0.6) (layer "F.Cu") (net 5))
 (segment (start 186.0739 69.4501) (end 186.0739 73.2087) (width 0.6) (layer "F.Cu") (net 5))
 (segment (start 178.308 71.66) (end 178.392 71.66) (width 0.6) (layer "F.Cu") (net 5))
 (segment (start 178.492 69.633) (end 178.91 69.215) (width 0.6) (layer "F.Cu") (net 5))
 (segment (start 209.4174 73.3351) (end 209.264 73.3351) (width 0.4) (layer "F.Cu") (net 3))
 (segment (start 209.5484 73.2041) (end 209.4174 73.3351) (width 0.4) (layer "F.Cu") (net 3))
 (segment (start 209.264 84.836) (end 209.264 73.3351) (width 0.4) (layer "F.Cu") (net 3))
 (segment (start 207.232 86.868) (end 209.264 84.836) (width 0.4) (layer "F.Cu") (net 3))
 (segment (start 178.3819 65.5) (end 176.3179 67.564) (width 0.4) (layer "F.Cu") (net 8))
 (segment (start 171.6065 67.564) (end 171.4052 67.7653) (width 0.4) (layer "F.Cu") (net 8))
 (segment (start 179.832 65.5) (end 178.3819 65.5) (width 0.4) (layer "F.Cu") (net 8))
 (segment (start 176.3179 67.564) (end 171.6065 67.564) (width 0.4) (layer "F.Cu") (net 8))
 (segment (start 202.692 75.5194) (end 202.692 69.667218) (width 0.4) (layer "F.Cu") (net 14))
 (segment (start 203.5714 76.3988) (end 202.692 75.5194) (width 0.4) (layer "F.Cu") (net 14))
 (segment (start 203.538418 68.8208) (end 205.3156 68.8208) (width 0.4) (layer "F.Cu") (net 14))
 (segment (start 205.1715 76.3988) (end 203.5714 76.3988) (width 0.4) (layer "F.Cu") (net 14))
 (segment (start 202.692 69.667218) (end 203.538418 68.8208) (width 0.4) (layer "F.Cu") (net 14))
 (segment (start 200.2656 71.3608) (end 200.2656 75.0847) (width 0.4) (layer "F.Cu") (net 16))
 (segment (start 200.2656 75.0847) (end 200.2215 75.1288) (width 0.4) (layer "F.Cu") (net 16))
 (segment (start 205.264 75.0363) (end 205.1715 75.1288) (width 0.4) (layer "F.Cu") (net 15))
 (segment (start 205.3156 73.2835) (end 205.264 73.3351) (width 0.4) (layer "F.Cu") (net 15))
 (segment (start 205.264 73.3351) (end 205.264 75.0363) (width 0.4) (layer "F.Cu") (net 15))
 (segment (start 205.3156 71.3608) (end 205.3156 73.2835) (width 0.4) (layer "F.Cu") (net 15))
 (segment (start 189.879222 76.674122) (end 197.293322 76.674122) (width 0.4) (layer "F.Cu") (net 6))
 (segment (start 197.293322 76.674122) (end 198.288 77.6688) (width 0.4) (layer "F.Cu") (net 6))
 (segment (start 198.288 77.6688) (end 200.2215 77.6688) (width 0.4) (layer "F.Cu") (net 6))
 (segment (start 188.6139 73.2087) (end 188.6139 75.4088) (width 0.4) (layer "F.Cu") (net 6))
 (segment (start 188.6139 75.4088) (end 189.879222 76.674122) (width 0.4) (layer "F.Cu") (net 6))
 (segment (start 198.3188 76.3988) (end 197.612 75.692) (width 0.4) (layer "F.Cu") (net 7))
 (segment (start 191.7992 75.692) (end 191.1539 75.0467) (width 0.4) (layer "F.Cu") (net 7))
 (segment (start 197.612 75.692) (end 191.7992 75.692) (width 0.4) (layer "F.Cu") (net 7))
 (segment (start 200.2215 76.3988) (end 198.3188 76.3988) (width 0.4) (layer "F.Cu") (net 7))
 (segment (start 191.1539 75.0467) (end 191.1539 73.2087) (width 0.4) (layer "F.Cu") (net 7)))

